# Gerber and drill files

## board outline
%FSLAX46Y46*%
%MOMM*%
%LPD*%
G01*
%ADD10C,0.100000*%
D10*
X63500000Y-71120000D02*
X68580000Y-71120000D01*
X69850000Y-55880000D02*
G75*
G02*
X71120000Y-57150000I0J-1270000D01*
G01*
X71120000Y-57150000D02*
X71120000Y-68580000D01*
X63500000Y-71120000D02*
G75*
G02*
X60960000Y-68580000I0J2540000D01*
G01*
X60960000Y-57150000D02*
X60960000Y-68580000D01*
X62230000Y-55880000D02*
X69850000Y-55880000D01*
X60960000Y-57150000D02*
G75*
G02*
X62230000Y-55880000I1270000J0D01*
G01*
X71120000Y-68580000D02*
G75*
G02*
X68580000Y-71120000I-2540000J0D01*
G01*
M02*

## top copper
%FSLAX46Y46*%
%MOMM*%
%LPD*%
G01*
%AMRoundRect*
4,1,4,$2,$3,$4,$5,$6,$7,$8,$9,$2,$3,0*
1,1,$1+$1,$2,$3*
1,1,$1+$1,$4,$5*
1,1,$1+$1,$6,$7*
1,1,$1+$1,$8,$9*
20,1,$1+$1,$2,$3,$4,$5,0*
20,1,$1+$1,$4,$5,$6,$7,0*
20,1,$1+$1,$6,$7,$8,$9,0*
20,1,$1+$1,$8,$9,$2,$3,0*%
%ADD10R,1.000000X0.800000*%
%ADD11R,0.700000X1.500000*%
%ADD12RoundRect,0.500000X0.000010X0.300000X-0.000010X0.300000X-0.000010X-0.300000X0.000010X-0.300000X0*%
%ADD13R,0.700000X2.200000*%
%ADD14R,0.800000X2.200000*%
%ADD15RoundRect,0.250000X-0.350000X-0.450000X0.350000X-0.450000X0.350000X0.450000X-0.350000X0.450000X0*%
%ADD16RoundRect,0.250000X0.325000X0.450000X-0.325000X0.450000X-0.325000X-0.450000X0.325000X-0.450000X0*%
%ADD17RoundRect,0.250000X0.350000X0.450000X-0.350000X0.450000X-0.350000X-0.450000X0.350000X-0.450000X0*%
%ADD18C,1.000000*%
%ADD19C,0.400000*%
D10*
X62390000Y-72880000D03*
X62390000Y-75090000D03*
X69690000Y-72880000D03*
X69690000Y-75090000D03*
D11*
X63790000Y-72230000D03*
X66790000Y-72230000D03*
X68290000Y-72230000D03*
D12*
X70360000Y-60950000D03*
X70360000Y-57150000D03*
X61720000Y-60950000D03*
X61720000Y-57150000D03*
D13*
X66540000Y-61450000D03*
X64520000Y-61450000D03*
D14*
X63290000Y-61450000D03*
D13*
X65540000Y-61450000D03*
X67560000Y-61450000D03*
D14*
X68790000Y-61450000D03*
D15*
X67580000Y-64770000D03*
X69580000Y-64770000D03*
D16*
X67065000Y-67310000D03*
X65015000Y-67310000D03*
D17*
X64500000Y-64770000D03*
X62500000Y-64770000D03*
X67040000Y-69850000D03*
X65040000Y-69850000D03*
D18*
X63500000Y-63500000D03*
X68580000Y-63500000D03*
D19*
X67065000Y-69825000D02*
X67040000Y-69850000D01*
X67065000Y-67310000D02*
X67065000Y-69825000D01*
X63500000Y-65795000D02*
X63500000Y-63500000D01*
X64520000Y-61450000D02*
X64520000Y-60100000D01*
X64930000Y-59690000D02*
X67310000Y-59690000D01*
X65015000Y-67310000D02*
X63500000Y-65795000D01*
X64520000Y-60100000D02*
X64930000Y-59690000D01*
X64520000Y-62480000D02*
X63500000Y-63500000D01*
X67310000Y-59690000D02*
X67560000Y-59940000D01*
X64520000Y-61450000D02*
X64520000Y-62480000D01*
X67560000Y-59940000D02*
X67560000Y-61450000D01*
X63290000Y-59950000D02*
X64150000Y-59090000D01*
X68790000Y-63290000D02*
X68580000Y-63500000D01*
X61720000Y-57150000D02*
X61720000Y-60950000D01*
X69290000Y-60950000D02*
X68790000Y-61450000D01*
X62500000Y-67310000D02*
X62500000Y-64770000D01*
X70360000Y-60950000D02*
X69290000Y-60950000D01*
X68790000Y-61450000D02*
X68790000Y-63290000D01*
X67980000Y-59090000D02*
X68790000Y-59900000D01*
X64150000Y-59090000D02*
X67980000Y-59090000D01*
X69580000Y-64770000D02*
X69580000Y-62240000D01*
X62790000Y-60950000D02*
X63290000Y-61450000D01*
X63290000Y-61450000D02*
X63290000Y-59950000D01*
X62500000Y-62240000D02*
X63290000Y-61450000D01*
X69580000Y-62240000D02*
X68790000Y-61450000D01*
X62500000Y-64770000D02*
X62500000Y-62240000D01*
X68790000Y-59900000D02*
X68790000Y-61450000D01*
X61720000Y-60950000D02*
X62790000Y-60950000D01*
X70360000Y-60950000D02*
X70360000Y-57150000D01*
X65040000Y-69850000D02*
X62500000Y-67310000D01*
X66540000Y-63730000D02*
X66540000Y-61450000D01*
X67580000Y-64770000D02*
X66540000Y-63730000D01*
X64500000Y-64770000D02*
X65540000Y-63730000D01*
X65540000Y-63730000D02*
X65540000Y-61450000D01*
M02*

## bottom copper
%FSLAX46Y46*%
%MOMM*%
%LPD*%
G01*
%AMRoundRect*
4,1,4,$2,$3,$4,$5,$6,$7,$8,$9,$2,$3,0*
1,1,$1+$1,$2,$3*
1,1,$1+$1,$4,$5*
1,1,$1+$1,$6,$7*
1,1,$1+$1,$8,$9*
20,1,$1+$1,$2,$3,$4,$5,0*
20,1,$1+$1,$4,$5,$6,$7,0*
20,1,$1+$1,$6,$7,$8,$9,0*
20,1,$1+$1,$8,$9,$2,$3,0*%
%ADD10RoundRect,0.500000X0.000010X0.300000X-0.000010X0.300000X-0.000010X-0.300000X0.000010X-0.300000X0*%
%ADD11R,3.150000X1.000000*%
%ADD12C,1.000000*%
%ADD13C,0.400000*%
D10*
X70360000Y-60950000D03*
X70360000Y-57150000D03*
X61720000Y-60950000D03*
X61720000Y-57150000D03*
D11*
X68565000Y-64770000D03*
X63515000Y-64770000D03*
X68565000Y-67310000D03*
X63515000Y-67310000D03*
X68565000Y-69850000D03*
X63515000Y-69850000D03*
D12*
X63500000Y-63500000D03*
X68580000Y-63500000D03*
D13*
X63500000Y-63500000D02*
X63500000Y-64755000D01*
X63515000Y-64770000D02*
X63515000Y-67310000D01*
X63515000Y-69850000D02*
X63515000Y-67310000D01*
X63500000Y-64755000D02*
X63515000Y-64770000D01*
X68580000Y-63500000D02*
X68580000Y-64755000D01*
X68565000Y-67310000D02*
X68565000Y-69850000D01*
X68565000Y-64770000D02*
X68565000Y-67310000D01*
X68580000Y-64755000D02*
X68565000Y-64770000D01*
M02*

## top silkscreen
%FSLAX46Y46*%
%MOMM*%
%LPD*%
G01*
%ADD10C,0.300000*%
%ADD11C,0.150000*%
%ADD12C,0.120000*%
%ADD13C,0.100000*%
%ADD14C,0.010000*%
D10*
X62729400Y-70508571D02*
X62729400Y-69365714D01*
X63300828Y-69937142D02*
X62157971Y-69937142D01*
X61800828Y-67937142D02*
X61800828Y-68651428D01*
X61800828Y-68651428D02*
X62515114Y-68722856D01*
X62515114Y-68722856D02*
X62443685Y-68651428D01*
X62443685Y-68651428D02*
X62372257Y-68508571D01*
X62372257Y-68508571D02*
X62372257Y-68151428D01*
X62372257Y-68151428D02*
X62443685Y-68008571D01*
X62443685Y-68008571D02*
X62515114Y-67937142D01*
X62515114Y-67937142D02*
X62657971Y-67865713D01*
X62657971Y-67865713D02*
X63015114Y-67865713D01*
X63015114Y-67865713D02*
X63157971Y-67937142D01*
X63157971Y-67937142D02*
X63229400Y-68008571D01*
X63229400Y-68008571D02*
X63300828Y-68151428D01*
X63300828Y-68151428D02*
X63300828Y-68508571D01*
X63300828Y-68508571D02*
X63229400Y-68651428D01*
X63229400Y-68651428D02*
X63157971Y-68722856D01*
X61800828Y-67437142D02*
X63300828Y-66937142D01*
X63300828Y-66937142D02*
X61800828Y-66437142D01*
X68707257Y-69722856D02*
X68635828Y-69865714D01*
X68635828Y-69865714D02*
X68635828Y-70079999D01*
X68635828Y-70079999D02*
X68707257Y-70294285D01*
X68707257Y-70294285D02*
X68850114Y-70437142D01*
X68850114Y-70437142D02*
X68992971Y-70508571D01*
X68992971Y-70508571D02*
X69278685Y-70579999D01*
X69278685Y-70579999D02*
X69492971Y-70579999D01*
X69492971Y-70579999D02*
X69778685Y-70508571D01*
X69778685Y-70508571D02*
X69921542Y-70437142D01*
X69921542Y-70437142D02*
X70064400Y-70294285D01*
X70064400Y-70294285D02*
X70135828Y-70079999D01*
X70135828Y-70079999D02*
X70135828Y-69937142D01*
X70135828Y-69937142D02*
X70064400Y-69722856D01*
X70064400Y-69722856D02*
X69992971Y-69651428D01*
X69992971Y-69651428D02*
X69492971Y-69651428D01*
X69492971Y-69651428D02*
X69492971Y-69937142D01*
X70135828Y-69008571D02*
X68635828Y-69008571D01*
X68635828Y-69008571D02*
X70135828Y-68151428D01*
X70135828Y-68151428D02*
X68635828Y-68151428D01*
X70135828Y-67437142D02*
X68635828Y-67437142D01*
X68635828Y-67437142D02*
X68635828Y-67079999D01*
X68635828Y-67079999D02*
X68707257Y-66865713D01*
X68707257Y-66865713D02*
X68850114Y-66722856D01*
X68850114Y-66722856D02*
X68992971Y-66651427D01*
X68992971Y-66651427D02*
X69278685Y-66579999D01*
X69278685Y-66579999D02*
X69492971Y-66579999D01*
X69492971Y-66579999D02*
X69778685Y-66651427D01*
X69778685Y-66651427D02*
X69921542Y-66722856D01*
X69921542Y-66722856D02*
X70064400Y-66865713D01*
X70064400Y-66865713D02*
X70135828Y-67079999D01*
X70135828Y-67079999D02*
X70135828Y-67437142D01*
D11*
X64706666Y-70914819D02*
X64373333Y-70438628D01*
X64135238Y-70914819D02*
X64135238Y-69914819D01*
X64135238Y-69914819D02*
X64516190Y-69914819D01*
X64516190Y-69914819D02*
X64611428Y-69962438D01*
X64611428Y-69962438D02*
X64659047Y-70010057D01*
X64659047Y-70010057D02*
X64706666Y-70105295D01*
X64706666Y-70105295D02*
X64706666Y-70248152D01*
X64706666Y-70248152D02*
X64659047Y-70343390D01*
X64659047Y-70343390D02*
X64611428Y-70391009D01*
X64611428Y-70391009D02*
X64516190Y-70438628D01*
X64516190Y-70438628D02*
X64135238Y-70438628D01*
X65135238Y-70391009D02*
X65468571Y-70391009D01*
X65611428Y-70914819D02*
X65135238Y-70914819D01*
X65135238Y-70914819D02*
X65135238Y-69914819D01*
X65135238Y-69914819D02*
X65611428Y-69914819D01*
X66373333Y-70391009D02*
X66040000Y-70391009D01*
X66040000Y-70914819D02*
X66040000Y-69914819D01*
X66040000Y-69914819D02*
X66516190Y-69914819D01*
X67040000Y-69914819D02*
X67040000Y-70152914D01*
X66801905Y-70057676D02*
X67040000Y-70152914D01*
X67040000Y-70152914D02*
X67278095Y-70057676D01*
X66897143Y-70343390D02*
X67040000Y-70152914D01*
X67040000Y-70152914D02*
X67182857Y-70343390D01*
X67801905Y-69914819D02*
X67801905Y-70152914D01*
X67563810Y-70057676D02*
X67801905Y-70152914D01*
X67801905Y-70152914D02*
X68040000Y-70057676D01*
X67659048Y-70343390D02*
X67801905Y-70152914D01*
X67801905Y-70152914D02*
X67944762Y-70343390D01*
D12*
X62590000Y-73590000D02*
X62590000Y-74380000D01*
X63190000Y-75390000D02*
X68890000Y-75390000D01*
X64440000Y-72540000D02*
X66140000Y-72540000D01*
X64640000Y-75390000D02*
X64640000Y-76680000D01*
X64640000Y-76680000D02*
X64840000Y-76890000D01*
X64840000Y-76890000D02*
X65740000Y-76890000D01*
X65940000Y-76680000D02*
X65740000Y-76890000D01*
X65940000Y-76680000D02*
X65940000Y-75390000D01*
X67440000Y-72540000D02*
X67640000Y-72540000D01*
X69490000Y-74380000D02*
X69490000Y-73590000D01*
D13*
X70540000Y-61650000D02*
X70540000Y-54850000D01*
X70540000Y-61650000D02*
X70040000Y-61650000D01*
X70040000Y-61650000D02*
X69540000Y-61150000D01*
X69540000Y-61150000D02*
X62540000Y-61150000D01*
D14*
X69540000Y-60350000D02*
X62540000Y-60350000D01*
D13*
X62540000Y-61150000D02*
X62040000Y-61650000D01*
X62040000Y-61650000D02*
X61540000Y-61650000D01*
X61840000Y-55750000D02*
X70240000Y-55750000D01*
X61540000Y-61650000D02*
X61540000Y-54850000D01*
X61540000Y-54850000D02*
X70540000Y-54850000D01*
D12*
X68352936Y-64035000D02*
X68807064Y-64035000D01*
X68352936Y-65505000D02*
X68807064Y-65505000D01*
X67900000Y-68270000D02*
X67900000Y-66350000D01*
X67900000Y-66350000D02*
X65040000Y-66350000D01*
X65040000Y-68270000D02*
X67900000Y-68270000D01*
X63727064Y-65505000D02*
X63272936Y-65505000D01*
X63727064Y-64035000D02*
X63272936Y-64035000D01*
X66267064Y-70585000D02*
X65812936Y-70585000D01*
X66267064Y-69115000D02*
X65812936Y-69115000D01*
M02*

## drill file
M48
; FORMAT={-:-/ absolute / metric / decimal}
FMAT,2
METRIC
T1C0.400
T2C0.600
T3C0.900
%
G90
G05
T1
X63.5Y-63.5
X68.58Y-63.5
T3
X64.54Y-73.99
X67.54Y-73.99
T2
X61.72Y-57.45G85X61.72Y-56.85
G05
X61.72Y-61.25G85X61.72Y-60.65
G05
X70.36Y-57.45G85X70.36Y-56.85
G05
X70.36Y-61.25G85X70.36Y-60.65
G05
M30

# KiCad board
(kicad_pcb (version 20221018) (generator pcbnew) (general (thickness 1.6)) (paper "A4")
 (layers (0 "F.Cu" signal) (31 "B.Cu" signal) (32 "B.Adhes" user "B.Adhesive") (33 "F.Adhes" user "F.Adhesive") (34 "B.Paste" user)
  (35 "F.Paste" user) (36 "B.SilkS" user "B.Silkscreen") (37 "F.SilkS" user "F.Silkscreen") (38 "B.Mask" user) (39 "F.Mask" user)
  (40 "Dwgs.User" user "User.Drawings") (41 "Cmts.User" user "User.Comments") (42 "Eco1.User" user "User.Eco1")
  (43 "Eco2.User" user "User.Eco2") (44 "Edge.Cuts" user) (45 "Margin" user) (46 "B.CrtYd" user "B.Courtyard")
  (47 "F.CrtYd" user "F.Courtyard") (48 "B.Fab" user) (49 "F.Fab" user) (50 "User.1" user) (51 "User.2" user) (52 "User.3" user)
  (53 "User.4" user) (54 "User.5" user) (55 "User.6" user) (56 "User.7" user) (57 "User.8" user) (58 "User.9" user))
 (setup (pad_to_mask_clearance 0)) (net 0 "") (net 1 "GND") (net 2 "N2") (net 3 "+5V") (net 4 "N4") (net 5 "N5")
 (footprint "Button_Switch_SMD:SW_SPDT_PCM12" (layer "F.Cu") (at 66.04 73.66)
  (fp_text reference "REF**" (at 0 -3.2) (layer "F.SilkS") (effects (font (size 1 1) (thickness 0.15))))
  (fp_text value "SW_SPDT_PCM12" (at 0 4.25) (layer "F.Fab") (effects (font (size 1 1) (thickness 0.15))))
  (fp_line (start -3.45 -0.07) (end -3.45 0.72) (stroke (width 0.12) (type solid)) (layer "F.SilkS"))
  (fp_line (start -2.85 1.73) (end 2.85 1.73) (stroke (width 0.12) (type solid)) (layer "F.SilkS"))
  (fp_line (start -1.6 -1.12) (end 0.1 -1.12) (stroke (width 0.12) (type solid)) (layer "F.SilkS"))
  (fp_line (start -1.4 1.73) (end -1.4 3.02) (stroke (width 0.12) (type solid)) (layer "F.SilkS"))
  (fp_line (start -1.4 3.02) (end -1.2 3.23) (stroke (width 0.12) (type solid)) (layer "F.SilkS"))
  (fp_line (start -1.2 3.23) (end -0.3 3.23) (stroke (width 0.12) (type solid)) (layer "F.SilkS"))
  (fp_line (start -0.1 3.02) (end -0.3 3.23) (stroke (width 0.12) (type solid)) (layer "F.SilkS"))
  (fp_line (start -0.1 3.02) (end -0.1 1.73) (stroke (width 0.12) (type solid)) (layer "F.SilkS"))
  (fp_line (start 1.4 -1.12) (end 1.6 -1.12) (stroke (width 0.12) (type solid)) (layer "F.SilkS"))
  (fp_line (start 3.45 0.72) (end 3.45 -0.07) (stroke (width 0.12) (type solid)) (layer "F.SilkS"))
  (pad "" smd rect (at -3.65 -0.78) (size 1 0.8) (layers "F.Cu" "F.Paste" "F.Mask"))
  (pad "" smd rect (at -3.65 1.43) (size 1 0.8) (layers "F.Cu" "F.Paste" "F.Mask"))
  (pad "" np_thru_hole circle (at -1.5 0.33) (size 0.9 0.9) (drill 0.9) (layers "*.Cu" "*.Mask"))
  (pad "" np_thru_hole circle (at 1.5 0.33) (size 0.9 0.9) (drill 0.9) (layers "*.Cu" "*.Mask"))
  (pad "" smd rect (at 3.65 -0.78) (size 1 0.8) (layers "F.Cu" "F.Paste" "F.Mask"))
  (pad "" smd rect (at 3.65 1.43) (size 1 0.8) (layers "F.Cu" "F.Paste" "F.Mask"))
  (pad "1" smd rect (at -2.25 -1.43) (size 0.7 1.5) (layers "F.Cu" "F.Paste" "F.Mask"))
  (pad "2" smd rect (at 0.75 -1.43) (size 0.7 1.5) (layers "F.Cu" "F.Paste" "F.Mask"))
  (pad "3" smd rect (at 2.25 -1.43) (size 0.7 1.5) (layers "F.Cu" "F.Paste" "F.Mask")))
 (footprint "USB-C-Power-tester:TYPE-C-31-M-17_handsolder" (layer "F.Cu") (at 66.04 57.15 180)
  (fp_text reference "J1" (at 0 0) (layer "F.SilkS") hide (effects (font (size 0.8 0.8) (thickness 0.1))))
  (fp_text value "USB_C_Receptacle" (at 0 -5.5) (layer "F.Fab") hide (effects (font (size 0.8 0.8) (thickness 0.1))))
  (fp_line (start -4.5 -4.5) (end -4.5 2.3) (stroke (width 0.1) (type solid)) (layer "F.SilkS"))
  (fp_line (start -4.5 -4.5) (end -4 -4.5) (stroke (width 0.1) (type solid)) (layer "F.SilkS"))
  (fp_line (start -4 -4.5) (end -3.5 -4) (stroke (width 0.1) (type solid)) (layer "F.SilkS"))
  (fp_line (start -3.5 -4) (end 3.5 -4) (stroke (width 0.1) (type solid)) (layer "F.SilkS"))
  (fp_line (start -3.5 -3.2) (end 3.5 -3.2) (stroke (width 0.01) (type solid)) (layer "F.SilkS"))
  (fp_line (start 3.5 -4) (end 4 -4.5) (stroke (width 0.1) (type solid)) (layer "F.SilkS"))
  (fp_line (start 4 -4.5) (end 4.5 -4.5) (stroke (width 0.1) (type solid)) (layer "F.SilkS"))
  (fp_line (start 4.2 1.4) (end -4.2 1.4) (stroke (width 0.1) (type solid)) (layer "F.SilkS"))
  (fp_line (start 4.5 -4.5) (end 4.5 2.3) (stroke (width 0.1) (type solid)) (layer "F.SilkS"))
  (fp_line (start 4.5 2.3) (end -4.5 2.3) (stroke (width 0.1) (type solid)) (layer "F.SilkS"))
  (pad "1" thru_hole roundrect (at -4.32 -3.8 180) (size 1 1.6) (drill oval 0.6 1.2) (layers "*.Cu" "*.Mask") (roundrect_rratio 0.5)
   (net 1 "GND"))
  (pad "1" thru_hole roundrect (at -4.32 0 180) (size 1 1.6) (drill oval 0.6 1.2) (layers "*.Cu" "*.Mask") (roundrect_rratio 0.5)
   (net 1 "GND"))
  (pad "1" thru_hole roundrect (at 4.32 -3.8 180) (size 1 1.6) (drill oval 0.6 1.2) (layers "*.Cu" "*.Mask") (roundrect_rratio 0.5)
   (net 1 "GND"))
  (pad "1" thru_hole roundrect (at 4.32 0 180) (size 1 1.6) (drill oval 0.6 1.2) (layers "*.Cu" "*.Mask") (roundrect_rratio 0.5)
   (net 1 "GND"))
  (pad "A5" smd rect (at -0.5 -4.3 180) (size 0.7 2.2) (layers "F.Cu" "F.Paste" "F.Mask") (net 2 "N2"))
  (pad "A9" smd rect (at 1.52 -4.3 180) (size 0.7 2.2) (layers "F.Cu" "F.Paste" "F.Mask") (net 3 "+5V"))
  (pad "A12" smd rect (at 2.75 -4.3 180) (size 0.8 2.2) (layers "F.Cu" "F.Paste" "F.Mask") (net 1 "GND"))
  (pad "B5" smd rect (at 0.5 -4.3 180) (size 0.7 2.2) (layers "F.Cu" "F.Paste" "F.Mask") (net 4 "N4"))
  (pad "B9" smd rect (at -1.52 -4.3 180) (size 0.7 2.2) (layers "F.Cu" "F.Paste" "F.Mask") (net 3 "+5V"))
  (pad "B12" smd rect (at -2.75 -4.3 180) (size 0.8 2.2) (layers "F.Cu" "F.Paste" "F.Mask") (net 1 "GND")))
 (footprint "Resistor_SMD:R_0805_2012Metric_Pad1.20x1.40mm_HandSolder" (layer "F.Cu") (at 68.58 64.77)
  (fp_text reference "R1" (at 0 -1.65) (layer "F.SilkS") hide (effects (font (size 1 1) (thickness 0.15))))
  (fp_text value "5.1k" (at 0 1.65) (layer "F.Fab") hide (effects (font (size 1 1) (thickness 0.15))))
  (fp_line (start -0.227064 -0.735) (end 0.227064 -0.735) (stroke (width 0.12) (type solid)) (layer "F.SilkS"))
  (fp_line (start -0.227064 0.735) (end 0.227064 0.735) (stroke (width 0.12) (type solid)) (layer "F.SilkS"))
  (pad "1" smd roundrect (at -1 0) (size 1.2 1.4) (layers "F.Cu" "F.Paste" "F.Mask") (roundrect_rratio 0.208333) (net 2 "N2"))
  (pad "2" smd roundrect (at 1 0) (size 1.2 1.4) (layers "F.Cu" "F.Paste" "F.Mask") (roundrect_rratio 0.208333) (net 1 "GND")))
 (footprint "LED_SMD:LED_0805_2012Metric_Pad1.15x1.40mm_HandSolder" (layer "F.Cu") (at 66.04 67.31 180)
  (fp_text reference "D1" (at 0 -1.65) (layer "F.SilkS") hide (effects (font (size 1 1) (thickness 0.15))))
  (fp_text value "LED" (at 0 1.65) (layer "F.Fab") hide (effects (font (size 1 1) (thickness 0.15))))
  (fp_line (start -1.86 -0.96) (end -1.86 0.96) (stroke (width 0.12) (type solid)) (layer "F.SilkS"))
  (fp_line (start -1.86 0.96) (end 1 0.96) (stroke (width 0.12) (type solid)) (layer "F.SilkS"))
  (fp_line (start 1 -0.96) (end -1.86 -0.96) (stroke (width 0.12) (type solid)) (layer "F.SilkS"))
  (pad "1" smd roundrect (at -1.025 0 180) (size 1.15 1.4) (layers "F.Cu" "F.Paste" "F.Mask") (roundrect_rratio 0.217391) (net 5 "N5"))
  (pad "2" smd roundrect (at 1.025 0 180) (size 1.15 1.4) (layers "F.Cu" "F.Paste" "F.Mask") (roundrect_rratio 0.217391) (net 3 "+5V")))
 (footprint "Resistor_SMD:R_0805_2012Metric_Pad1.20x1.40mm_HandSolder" (layer "F.Cu") (at 63.5 64.77 180)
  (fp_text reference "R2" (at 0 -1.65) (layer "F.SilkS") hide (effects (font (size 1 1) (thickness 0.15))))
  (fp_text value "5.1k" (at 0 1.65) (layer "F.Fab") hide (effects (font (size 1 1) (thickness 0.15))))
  (fp_line (start -0.227064 -0.735) (end 0.227064 -0.735) (stroke (width 0.12) (type solid)) (layer "F.SilkS"))
  (fp_line (start -0.227064 0.735) (end 0.227064 0.735) (stroke (width 0.12) (type solid)) (layer "F.SilkS"))
  (pad "1" smd roundrect (at -1 0 180) (size 1.2 1.4) (layers "F.Cu" "F.Paste" "F.Mask") (roundrect_rratio 0.208333) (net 4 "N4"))
  (pad "2" smd roundrect (at 1 0 180) (size 1.2 1.4) (layers "F.Cu" "F.Paste" "F.Mask") (roundrect_rratio 0.208333) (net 1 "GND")))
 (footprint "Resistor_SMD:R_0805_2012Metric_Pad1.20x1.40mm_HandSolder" (layer "F.Cu") (at 66.04 69.85 180)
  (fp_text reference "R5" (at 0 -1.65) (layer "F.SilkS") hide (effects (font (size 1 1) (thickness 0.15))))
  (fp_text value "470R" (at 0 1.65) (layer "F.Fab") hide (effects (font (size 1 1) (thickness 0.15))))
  (fp_line (start -0.227064 -0.735) (end 0.227064 -0.735) (stroke (width 0.12) (type solid)) (layer "F.SilkS"))
  (fp_line (start -0.227064 0.735) (end 0.227064 0.735) (stroke (width 0.12) (type solid)) (layer "F.SilkS"))
  (pad "1" smd roundrect (at -1 0 180) (size 1.2 1.4) (layers "F.Cu" "F.Paste" "F.Mask") (roundrect_rratio 0.208333) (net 5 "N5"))
  (pad "2" smd roundrect (at 1 0 180) (size 1.2 1.4) (layers "F.Cu" "F.Paste" "F.Mask") (roundrect_rratio 0.208333) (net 1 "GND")))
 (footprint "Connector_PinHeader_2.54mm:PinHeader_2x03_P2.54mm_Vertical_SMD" (layer "B.Cu") (at 66.04 67.31 180)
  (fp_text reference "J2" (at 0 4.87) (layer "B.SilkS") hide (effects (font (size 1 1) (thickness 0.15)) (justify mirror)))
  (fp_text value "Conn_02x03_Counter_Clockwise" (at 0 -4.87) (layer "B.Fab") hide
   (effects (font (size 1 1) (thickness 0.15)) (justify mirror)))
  (pad "1" smd rect (at -2.525 2.54 180) (size 3.15 1) (layers "B.Cu" "B.Paste" "B.Mask") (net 1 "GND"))
  (pad "2" smd rect (at 2.525 2.54 180) (size 3.15 1) (layers "B.Cu" "B.Paste" "B.Mask") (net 3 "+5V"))
  (pad "3" smd rect (at -2.525 0 180) (size 3.15 1) (layers "B.Cu" "B.Paste" "B.Mask") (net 1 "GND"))
  (pad "4" smd rect (at 2.525 0 180) (size 3.15 1) (layers "B.Cu" "B.Paste" "B.Mask") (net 3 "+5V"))
  (pad "5" smd rect (at -2.525 -2.54 180) (size 3.15 1) (layers "B.Cu" "B.Paste" "B.Mask") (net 1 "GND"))
  (pad "6" smd rect (at 2.525 -2.54 180) (size 3.15 1) (layers "B.Cu" "B.Paste" "B.Mask") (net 3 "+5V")))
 (gr_line (start 63.5 71.12) (end 68.58 71.12) (stroke (width 0.1) (type default)) (layer "Edge.Cuts"))
 (gr_arc (start 69.85 55.88) (mid 70.748026 56.251974) (end 71.12 57.15) (stroke (width 0.1) (type default)) (layer "Edge.Cuts"))
 (gr_line (start 71.12 57.15) (end 71.12 68.58) (stroke (width 0.1) (type default)) (layer "Edge.Cuts"))
 (gr_arc (start 63.5 71.12) (mid 61.703949 70.376051) (end 60.96 68.58) (stroke (width 0.1) (type default)) (layer "Edge.Cuts"))
 (gr_line (start 60.96 57.15) (end 60.96 68.58) (stroke (width 0.1) (type default)) (layer "Edge.Cuts"))
 (gr_line (start 62.23 55.88) (end 69.85 55.88) (stroke (width 0.1) (type default)) (layer "Edge.Cuts"))
 (gr_arc (start 60.96 57.15) (mid 61.331974 56.251974) (end 62.23 55.88) (stroke (width 0.1) (type default)) (layer "Edge.Cuts"))
 (gr_arc (start 71.12 68.58) (mid 70.376051 70.376051) (end 68.58 71.12) (stroke (width 0.1) (type default)) (layer "Edge.Cuts"))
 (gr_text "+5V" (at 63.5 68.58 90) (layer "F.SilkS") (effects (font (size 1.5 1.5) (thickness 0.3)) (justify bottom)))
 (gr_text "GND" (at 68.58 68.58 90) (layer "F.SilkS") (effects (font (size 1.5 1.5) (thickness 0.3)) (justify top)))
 (segment (start 67.065 69.825) (end 67.04 69.85) (width 0.4) (layer "F.Cu") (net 5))
 (segment (start 67.065 67.31) (end 67.065 69.825) (width 0.4) (layer "F.Cu") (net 5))
 (segment (start 63.5 65.795) (end 63.5 63.5) (width 0.4) (layer "F.Cu") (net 3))
 (segment (start 64.52 61.45) (end 64.52 60.1) (width 0.4) (layer "F.Cu") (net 3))
 (segment (start 64.93 59.69) (end 67.31 59.69) (width 0.4) (layer "F.Cu") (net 3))
 (segment (start 65.015 67.31) (end 63.5 65.795) (width 0.4) (layer "F.Cu") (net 3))
 (segment (start 64.52 60.1) (end 64.93 59.69) (width 0.4) (layer "F.Cu") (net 3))
 (segment (start 64.52 62.48) (end 63.5 63.5) (width 0.4) (layer "F.Cu") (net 3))
 (segment (start 67.31 59.69) (end 67.56 59.94) (width 0.4) (layer "F.Cu") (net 3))
 (segment (start 64.52 61.45) (end 64.52 62.48) (width 0.4) (layer "F.Cu") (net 3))
 (segment (start 67.56 59.94) (end 67.56 61.45) (width 0.4) (layer "F.Cu") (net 3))
 (via (at 63.5 63.5) (size 1) (drill 0.4) (layers "F.Cu" "B.Cu") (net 3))
 (segment (start 63.5 63.5) (end 63.5 64.755) (width 0.4) (layer "B.Cu") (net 3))
 (segment (start 63.515 64.77) (end 63.515 67.31) (width 0.4) (layer "B.Cu") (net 3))
 (segment (start 63.515 69.85) (end 63.515 67.31) (width 0.4) (layer "B.Cu") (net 3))
 (segment (start 63.5 64.755) (end 63.515 64.77) (width 0.4) (layer "B.Cu") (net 3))
 (segment (start 63.29 59.95) (end 64.15 59.09) (width 0.4) (layer "F.Cu") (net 1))
 (segment (start 68.79 63.29) (end 68.58 63.5) (width 0.4) (layer "F.Cu") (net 1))
 (segment (start 61.72 57.15) (end 61.72 60.95) (width 0.4) (layer "F.Cu") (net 1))
 (segment (start 69.29 60.95) (end 68.79 61.45) (width 0.4) (layer "F.Cu") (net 1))
 (segment (start 62.5 67.31) (end 62.5 64.77) (width 0.4) (layer "F.Cu") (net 1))
 (segment (start 70.36 60.95) (end 69.29 60.95) (width 0.4) (layer "F.Cu") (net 1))
 (segment (start 68.79 61.45) (end 68.79 63.29) (width 0.4) (layer "F.Cu") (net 1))
 (segment (start 67.98 59.09) (end 68.79 59.9) (width 0.4) (layer "F.Cu") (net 1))
 (segment (start 64.15 59.09) (end 67.98 59.09) (width 0.4) (layer "F.Cu") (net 1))
 (segment (start 69.58 64.77) (end 69.58 62.24) (width 0.4) (layer "F.Cu") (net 1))
 (segment (start 62.79 60.95) (end 63.29 61.45) (width 0.4) (layer "F.Cu") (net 1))
 (segment (start 63.29 61.45) (end 63.29 59.95) (width 0.4) (layer "F.Cu") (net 1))
 (segment (start 62.5 62.24) (end 63.29 61.45) (width 0.4) (layer "F.Cu") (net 1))
 (segment (start 69.58 62.24) (end 68.79 61.45) (width 0.4) (layer "F.Cu") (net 1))
 (segment (start 62.5 64.77) (end 62.5 62.24) (width 0.4) (layer "F.Cu") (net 1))
 (segment (start 68.79 59.9) (end 68.79 61.45) (width 0.4) (layer "F.Cu") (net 1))
 (segment (start 61.72 60.95) (end 62.79 60.95) (width 0.4) (layer "F.Cu") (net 1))
 (segment (start 70.36 60.95) (end 70.36 57.15) (width 0.4) (layer "F.Cu") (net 1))
 (segment (start 65.04 69.85) (end 62.5 67.31) (width 0.4) (layer "F.Cu") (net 1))
 (via (at 68.58 63.5) (size 1) (drill 0.4) (layers "F.Cu" "B.Cu") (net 1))
 (segment (start 68.58 63.5) (end 68.58 64.755) (width 0.4) (layer "B.Cu") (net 1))
 (segment (start 68.565 67.31) (end 68.565 69.85) (width 0.4) (layer "B.Cu") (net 1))
 (segment (start 68.565 64.77) (end 68.565 67.31) (width 0.4) (layer "B.Cu") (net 1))
 (segment (start 68.58 64.755) (end 68.565 64.77) (width 0.4) (layer "B.Cu") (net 1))
 (segment (start 66.54 63.73) (end 66.54 61.45) (width 0.4) (layer "F.Cu") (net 2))
 (segment (start 67.58 64.77) (end 66.54 63.73) (width 0.4) (layer "F.Cu") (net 2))
 (segment (start 64.5 64.77) (end 65.54 63.73) (width 0.4) (layer "F.Cu") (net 4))
 (segment (start 65.54 63.73) (end 65.54 61.45) (width 0.4) (layer "F.Cu") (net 4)))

